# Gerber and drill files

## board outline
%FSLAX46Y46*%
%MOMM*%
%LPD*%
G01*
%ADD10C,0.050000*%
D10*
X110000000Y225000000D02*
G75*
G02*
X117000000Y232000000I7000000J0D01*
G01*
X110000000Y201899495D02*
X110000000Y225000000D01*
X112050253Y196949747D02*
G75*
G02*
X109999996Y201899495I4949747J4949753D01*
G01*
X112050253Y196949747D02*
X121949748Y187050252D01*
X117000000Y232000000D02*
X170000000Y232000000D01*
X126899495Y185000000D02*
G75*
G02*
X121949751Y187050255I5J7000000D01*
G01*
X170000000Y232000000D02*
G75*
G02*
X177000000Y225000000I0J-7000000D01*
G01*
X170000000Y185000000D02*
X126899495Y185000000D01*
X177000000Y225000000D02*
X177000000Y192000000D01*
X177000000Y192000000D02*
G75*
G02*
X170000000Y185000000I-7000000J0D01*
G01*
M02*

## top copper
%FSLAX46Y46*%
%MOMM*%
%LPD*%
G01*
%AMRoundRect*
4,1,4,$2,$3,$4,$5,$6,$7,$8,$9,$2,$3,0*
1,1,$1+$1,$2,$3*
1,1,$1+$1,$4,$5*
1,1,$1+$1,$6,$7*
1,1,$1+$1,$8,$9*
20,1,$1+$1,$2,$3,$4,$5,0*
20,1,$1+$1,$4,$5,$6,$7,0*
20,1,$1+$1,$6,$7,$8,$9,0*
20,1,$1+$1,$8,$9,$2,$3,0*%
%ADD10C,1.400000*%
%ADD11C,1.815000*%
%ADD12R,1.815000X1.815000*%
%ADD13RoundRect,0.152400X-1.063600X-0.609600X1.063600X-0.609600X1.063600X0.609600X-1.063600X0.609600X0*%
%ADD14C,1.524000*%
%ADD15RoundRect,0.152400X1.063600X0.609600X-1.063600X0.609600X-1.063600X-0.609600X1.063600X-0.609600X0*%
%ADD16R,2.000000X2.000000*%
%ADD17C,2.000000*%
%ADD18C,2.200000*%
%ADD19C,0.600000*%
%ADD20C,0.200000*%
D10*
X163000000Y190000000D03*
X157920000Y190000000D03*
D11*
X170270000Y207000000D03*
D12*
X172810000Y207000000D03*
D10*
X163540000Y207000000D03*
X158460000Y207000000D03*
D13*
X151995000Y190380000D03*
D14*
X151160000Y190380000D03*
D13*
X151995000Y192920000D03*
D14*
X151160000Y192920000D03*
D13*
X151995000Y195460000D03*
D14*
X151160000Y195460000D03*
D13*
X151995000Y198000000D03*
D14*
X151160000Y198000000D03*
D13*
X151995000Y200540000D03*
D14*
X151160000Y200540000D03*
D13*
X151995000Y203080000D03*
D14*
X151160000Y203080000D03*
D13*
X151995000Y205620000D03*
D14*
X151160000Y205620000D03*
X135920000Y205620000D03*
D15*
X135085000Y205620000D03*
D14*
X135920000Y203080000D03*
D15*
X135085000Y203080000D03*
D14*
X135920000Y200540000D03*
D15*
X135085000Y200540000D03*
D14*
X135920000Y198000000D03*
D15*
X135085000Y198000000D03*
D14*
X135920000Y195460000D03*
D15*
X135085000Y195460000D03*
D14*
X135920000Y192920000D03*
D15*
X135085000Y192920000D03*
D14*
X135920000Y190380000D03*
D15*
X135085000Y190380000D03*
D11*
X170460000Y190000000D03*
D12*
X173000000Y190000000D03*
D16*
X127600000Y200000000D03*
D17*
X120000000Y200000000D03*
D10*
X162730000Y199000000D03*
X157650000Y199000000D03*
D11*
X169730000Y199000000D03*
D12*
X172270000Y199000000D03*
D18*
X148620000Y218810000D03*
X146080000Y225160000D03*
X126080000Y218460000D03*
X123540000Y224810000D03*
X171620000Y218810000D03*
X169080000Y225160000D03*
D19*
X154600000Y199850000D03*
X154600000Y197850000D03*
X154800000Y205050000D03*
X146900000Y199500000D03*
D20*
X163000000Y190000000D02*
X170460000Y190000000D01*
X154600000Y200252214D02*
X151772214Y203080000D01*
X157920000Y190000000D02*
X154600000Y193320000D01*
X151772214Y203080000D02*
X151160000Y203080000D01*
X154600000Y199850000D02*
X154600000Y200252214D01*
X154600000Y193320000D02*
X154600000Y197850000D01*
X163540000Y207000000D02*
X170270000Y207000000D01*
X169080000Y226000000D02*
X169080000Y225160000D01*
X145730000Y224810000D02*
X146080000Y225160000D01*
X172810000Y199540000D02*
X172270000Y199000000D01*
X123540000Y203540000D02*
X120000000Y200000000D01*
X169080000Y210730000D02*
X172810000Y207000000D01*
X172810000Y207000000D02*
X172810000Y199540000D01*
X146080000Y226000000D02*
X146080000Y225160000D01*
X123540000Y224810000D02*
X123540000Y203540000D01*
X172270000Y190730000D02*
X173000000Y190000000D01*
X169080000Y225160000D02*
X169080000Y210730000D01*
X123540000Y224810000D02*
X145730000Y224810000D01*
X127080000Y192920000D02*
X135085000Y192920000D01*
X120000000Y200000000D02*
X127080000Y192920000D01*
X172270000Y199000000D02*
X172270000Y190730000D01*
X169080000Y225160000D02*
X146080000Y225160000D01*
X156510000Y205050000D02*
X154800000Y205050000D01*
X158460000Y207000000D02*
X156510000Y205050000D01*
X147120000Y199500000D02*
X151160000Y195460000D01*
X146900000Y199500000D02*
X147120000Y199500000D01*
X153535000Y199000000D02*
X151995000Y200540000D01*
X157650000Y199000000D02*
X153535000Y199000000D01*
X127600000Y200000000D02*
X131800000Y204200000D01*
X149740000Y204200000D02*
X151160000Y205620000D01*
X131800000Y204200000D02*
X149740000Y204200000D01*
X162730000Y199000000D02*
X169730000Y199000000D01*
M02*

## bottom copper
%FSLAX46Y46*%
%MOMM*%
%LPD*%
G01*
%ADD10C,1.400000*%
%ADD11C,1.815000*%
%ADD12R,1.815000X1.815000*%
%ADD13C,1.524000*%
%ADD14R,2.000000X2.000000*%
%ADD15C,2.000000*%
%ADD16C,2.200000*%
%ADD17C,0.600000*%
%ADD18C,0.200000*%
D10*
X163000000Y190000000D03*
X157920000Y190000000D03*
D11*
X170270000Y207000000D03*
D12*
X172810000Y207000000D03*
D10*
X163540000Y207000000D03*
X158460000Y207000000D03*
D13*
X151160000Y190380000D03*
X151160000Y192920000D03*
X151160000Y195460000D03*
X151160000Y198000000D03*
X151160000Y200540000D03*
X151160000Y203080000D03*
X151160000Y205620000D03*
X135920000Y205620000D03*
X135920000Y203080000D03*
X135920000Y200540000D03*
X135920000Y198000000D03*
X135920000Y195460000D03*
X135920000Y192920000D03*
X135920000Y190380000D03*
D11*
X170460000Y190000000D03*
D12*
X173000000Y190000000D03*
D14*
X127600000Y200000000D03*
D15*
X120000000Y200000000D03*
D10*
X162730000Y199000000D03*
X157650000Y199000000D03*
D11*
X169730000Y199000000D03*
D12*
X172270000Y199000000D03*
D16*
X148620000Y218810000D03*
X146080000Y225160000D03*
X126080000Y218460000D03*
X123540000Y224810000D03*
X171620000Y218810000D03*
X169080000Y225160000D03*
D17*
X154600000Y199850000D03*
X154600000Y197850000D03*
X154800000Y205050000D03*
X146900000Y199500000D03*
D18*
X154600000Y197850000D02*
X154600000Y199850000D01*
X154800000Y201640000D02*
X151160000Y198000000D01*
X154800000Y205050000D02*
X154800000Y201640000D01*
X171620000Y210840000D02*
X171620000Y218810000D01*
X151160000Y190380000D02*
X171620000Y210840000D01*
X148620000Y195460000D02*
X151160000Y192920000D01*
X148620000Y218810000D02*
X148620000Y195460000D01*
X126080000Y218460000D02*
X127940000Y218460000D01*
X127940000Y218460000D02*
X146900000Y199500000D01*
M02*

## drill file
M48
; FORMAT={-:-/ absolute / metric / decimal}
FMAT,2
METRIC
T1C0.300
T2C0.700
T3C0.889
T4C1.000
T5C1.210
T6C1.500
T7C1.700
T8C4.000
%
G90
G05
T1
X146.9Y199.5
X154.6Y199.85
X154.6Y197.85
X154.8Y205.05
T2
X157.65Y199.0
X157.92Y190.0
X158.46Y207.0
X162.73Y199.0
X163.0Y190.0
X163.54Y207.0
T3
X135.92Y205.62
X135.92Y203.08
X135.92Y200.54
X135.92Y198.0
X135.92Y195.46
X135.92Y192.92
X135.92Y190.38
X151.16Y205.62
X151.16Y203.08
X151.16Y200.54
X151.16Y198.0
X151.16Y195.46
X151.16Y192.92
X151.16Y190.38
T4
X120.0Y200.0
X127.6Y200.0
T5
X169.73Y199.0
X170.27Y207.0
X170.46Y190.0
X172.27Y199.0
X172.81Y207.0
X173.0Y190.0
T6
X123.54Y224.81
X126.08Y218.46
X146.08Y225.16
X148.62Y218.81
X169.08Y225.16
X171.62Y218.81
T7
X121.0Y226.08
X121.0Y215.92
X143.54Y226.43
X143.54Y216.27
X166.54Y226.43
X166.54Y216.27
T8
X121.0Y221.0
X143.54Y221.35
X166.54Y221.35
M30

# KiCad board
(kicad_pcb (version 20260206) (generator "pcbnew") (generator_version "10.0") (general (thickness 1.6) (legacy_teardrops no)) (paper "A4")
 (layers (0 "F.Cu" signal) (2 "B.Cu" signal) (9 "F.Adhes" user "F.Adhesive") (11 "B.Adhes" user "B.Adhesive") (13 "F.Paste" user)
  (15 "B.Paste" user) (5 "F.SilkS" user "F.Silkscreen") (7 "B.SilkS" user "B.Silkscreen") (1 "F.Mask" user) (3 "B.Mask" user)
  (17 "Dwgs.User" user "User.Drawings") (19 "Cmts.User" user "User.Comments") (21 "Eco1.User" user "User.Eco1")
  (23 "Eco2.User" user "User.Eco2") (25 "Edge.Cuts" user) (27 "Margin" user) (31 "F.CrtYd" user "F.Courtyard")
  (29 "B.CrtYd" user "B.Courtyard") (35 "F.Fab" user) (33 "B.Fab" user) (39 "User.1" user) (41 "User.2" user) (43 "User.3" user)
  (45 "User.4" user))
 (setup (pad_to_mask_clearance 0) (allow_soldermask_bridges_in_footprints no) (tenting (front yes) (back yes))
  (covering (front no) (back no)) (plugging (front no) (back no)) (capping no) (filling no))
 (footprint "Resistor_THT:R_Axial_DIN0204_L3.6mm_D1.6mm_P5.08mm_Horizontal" (layer "F.Cu") (at 163 -190 180)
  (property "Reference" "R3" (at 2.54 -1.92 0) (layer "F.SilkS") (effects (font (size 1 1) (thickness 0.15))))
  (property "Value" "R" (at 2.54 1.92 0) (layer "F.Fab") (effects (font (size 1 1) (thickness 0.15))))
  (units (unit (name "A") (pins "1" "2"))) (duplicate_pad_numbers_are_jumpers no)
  (pad "1" thru_hole circle (at 0 0 180) (size 1.4 1.4) (drill 0.7) (layers "*.Cu" "*.Mask") (remove_unused_layers no) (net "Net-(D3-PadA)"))
  (pad "2" thru_hole circle (at 5.08 0 180) (size 1.4 1.4) (drill 0.7) (layers "*.Cu" "*.Mask") (remove_unused_layers no) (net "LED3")))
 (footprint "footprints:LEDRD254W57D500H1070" (layer "F.Cu") (at 171.54 -207 180)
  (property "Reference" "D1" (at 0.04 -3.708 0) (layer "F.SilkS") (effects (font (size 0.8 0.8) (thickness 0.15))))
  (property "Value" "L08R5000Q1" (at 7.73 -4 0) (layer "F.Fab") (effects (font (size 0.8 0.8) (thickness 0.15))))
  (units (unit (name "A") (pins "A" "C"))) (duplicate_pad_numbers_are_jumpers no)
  (pad "A" thru_hole circle (at 1.27 0 180) (size 1.815 1.815) (drill 1.21) (layers "*.Cu" "*.Mask") (remove_unused_layers no)
   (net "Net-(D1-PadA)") (solder_mask_margin 0.102))
  (pad "C" thru_hole rect (at -1.27 0 180) (size 1.815 1.815) (drill 1.21) (layers "*.Cu" "*.Mask") (remove_unused_layers no) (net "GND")
   (solder_mask_margin 0.102)))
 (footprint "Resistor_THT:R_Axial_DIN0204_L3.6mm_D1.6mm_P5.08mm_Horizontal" (layer "F.Cu") (at 163.54 -207 180)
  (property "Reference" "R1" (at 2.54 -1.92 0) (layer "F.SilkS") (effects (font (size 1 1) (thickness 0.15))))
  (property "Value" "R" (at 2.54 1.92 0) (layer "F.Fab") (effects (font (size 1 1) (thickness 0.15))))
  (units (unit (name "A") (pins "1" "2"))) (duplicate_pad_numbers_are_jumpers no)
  (pad "1" thru_hole circle (at 0 0 180) (size 1.4 1.4) (drill 0.7) (layers "*.Cu" "*.Mask") (remove_unused_layers no) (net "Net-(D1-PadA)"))
  (pad "2" thru_hole circle (at 5.08 0 180) (size 1.4 1.4) (drill 0.7) (layers "*.Cu" "*.Mask") (remove_unused_layers no) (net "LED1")))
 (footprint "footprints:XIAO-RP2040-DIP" (layer "F.Cu") (at 143.54 -198 -90)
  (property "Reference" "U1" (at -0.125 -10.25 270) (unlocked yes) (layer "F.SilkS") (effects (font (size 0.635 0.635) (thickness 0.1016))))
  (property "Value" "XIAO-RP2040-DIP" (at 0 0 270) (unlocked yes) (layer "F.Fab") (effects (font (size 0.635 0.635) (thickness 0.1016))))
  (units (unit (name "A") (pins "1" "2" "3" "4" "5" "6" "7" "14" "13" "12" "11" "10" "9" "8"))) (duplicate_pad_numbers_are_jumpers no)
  (pad "1" smd roundrect (at 7.62 -8.455) (size 2.432 1.524) (layers "F.Cu" "F.Mask") (roundrect_rratio 0.1) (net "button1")
   (thermal_bridge_angle 45))
  (pad "1" thru_hole circle (at 7.62 -7.62) (size 1.524 1.524) (drill 0.889) (layers "*.Cu" "*.Mask") (remove_unused_layers no)
   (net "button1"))
  (pad "2" smd roundrect (at 5.08 -8.455) (size 2.432 1.524) (layers "F.Cu" "F.Mask") (roundrect_rratio 0.1) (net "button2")
   (thermal_bridge_angle 45))
  (pad "2" thru_hole circle (at 5.08 -7.62) (size 1.524 1.524) (drill 0.889) (layers "*.Cu" "*.Mask") (remove_unused_layers no)
   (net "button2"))
  (pad "3" smd roundrect (at 2.54 -8.455) (size 2.432 1.524) (layers "F.Cu" "F.Mask") (roundrect_rratio 0.1) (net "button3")
   (thermal_bridge_angle 45))
  (pad "3" thru_hole circle (at 2.54 -7.62) (size 1.524 1.524) (drill 0.889) (layers "*.Cu" "*.Mask") (remove_unused_layers no)
   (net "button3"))
  (pad "4" smd roundrect (at 0 -8.455) (size 2.432 1.524) (layers "F.Cu" "F.Mask") (roundrect_rratio 0.1) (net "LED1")
   (thermal_bridge_angle 45))
  (pad "4" thru_hole circle (at 0 -7.62) (size 1.524 1.524) (drill 0.889) (layers "*.Cu" "*.Mask") (remove_unused_layers no) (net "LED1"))
  (pad "5" smd roundrect (at -2.54 -8.455) (size 2.432 1.524) (layers "F.Cu" "F.Mask") (roundrect_rratio 0.1) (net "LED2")
   (thermal_bridge_angle 45))
  (pad "5" thru_hole circle (at -2.54 -7.62) (size 1.524 1.524) (drill 0.889) (layers "*.Cu" "*.Mask") (remove_unused_layers no)
   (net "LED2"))
  (pad "6" smd roundrect (at -5.08 -8.455) (size 2.432 1.524) (layers "F.Cu" "F.Mask") (roundrect_rratio 0.1) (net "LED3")
   (thermal_bridge_angle 45))
  (pad "6" thru_hole circle (at -5.08 -7.62) (size 1.524 1.524) (drill 0.889) (layers "*.Cu" "*.Mask") (remove_unused_layers no)
   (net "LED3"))
  (pad "7" smd roundrect (at -7.62 -8.455) (size 2.432 1.524) (layers "F.Cu" "F.Mask") (roundrect_rratio 0.1) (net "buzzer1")
   (thermal_bridge_angle 45))
  (pad "7" thru_hole circle (at -7.62 -7.62) (size 1.524 1.524) (drill 0.889) (layers "*.Cu" "*.Mask") (remove_unused_layers no)
   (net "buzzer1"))
  (pad "8" thru_hole circle (at -7.62 7.62 180) (size 1.524 1.524) (drill 0.889) (layers "*.Cu" "*.Mask") (remove_unused_layers no)
   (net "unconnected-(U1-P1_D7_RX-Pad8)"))
  (pad "8" smd roundrect (at -7.62 8.455 180) (size 2.432 1.524) (layers "F.Cu" "F.Mask") (roundrect_rratio 0.1)
   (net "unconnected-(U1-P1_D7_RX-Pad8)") (thermal_bridge_angle 45))
  (pad "9" thru_hole circle (at -5.08 7.62 180) (size 1.524 1.524) (drill 0.889) (layers "*.Cu" "*.Mask") (remove_unused_layers no)
   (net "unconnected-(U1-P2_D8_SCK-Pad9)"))
  (pad "9" smd roundrect (at -5.08 8.455 180) (size 2.432 1.524) (layers "F.Cu" "F.Mask") (roundrect_rratio 0.1)
   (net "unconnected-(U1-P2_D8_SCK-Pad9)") (thermal_bridge_angle 45))
  (pad "10" thru_hole circle (at -2.54 7.62 180) (size 1.524 1.524) (drill 0.889) (layers "*.Cu" "*.Mask") (remove_unused_layers no)
   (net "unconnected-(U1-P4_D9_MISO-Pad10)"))
  (pad "10" smd roundrect (at -2.54 8.455 180) (size 2.432 1.524) (layers "F.Cu" "F.Mask") (roundrect_rratio 0.1)
   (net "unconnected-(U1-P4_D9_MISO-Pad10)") (thermal_bridge_angle 45))
  (pad "11" thru_hole circle (at 0 7.62 180) (size 1.524 1.524) (drill 0.889) (layers "*.Cu" "*.Mask") (remove_unused_layers no)
   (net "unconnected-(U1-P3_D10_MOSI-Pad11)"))
  (pad "11" smd roundrect (at 0 8.455 180) (size 2.432 1.524) (layers "F.Cu" "F.Mask") (roundrect_rratio 0.1)
   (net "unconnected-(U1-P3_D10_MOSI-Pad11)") (thermal_bridge_angle 45))
  (pad "12" thru_hole circle (at 2.54 7.62 180) (size 1.524 1.524) (drill 0.889) (layers "*.Cu" "*.Mask") (remove_unused_layers no)
   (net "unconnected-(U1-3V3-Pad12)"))
  (pad "12" smd roundrect (at 2.54 8.455 180) (size 2.432 1.524) (layers "F.Cu" "F.Mask") (roundrect_rratio 0.1)
   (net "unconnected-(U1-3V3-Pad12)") (thermal_bridge_angle 45))
  (pad "13" thru_hole circle (at 5.08 7.62 180) (size 1.524 1.524) (drill 0.889) (layers "*.Cu" "*.Mask") (remove_unused_layers no)
   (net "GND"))
  (pad "13" smd roundrect (at 5.08 8.455 180) (size 2.432 1.524) (layers "F.Cu" "F.Mask") (roundrect_rratio 0.1) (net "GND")
   (thermal_bridge_angle 45))
  (pad "14" thru_hole circle (at 7.62 7.62 180) (size 1.524 1.524) (drill 0.889) (layers "*.Cu" "*.Mask") (remove_unused_layers no)
   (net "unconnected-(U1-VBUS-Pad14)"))
  (pad "14" smd roundrect (at 7.62 8.455 180) (size 2.432 1.524) (layers "F.Cu" "F.Mask") (roundrect_rratio 0.1)
   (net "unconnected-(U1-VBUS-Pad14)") (thermal_bridge_angle 45)))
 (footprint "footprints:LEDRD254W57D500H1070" (layer "F.Cu") (at 171.73 -190 180)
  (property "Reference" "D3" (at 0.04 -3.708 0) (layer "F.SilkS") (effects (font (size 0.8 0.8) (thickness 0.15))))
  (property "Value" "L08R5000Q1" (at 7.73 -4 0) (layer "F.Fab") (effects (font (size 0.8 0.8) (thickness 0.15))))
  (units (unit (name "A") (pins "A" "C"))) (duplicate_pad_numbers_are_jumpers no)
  (pad "A" thru_hole circle (at 1.27 0 180) (size 1.815 1.815) (drill 1.21) (layers "*.Cu" "*.Mask") (remove_unused_layers no)
   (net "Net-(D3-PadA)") (solder_mask_margin 0.102))
  (pad "C" thru_hole rect (at -1.27 0 180) (size 1.815 1.815) (drill 1.21) (layers "*.Cu" "*.Mask") (remove_unused_layers no) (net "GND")
   (solder_mask_margin 0.102)))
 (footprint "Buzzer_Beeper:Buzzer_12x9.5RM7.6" (layer "F.Cu") (at 127.6 -200 180)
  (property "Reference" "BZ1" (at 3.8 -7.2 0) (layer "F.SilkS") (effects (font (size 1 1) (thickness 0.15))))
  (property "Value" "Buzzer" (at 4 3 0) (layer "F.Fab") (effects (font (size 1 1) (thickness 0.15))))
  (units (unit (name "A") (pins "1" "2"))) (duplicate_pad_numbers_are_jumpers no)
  (pad "1" thru_hole rect (at 0 0 180) (size 2 2) (drill 1) (layers "*.Cu" "*.Mask") (remove_unused_layers no) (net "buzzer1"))
  (pad "2" thru_hole circle (at 7.6 0 180) (size 2 2) (drill 1) (layers "*.Cu" "*.Mask") (remove_unused_layers no) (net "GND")))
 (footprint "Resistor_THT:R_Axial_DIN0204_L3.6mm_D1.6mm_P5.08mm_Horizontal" (layer "F.Cu") (at 162.73 -199 180)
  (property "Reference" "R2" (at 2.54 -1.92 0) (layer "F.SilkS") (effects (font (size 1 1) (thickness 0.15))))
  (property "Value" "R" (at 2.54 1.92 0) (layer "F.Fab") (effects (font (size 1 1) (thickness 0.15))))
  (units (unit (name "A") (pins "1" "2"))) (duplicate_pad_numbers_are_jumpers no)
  (pad "1" thru_hole circle (at 0 0 180) (size 1.4 1.4) (drill 0.7) (layers "*.Cu" "*.Mask") (remove_unused_layers no) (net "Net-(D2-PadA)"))
  (pad "2" thru_hole circle (at 5.08 0 180) (size 1.4 1.4) (drill 0.7) (layers "*.Cu" "*.Mask") (remove_unused_layers no) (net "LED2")))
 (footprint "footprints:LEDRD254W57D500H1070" (layer "F.Cu") (at 171 -199 180)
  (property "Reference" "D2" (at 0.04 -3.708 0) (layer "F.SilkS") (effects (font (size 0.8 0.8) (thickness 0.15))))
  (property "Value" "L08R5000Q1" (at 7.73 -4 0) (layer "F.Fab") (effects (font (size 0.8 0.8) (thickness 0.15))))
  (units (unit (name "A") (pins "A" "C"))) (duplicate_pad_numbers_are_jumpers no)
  (pad "A" thru_hole circle (at 1.27 0 180) (size 1.815 1.815) (drill 1.21) (layers "*.Cu" "*.Mask") (remove_unused_layers no)
   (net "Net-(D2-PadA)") (solder_mask_margin 0.102))
  (pad "C" thru_hole rect (at -1.27 0 180) (size 1.815 1.815) (drill 1.21) (layers "*.Cu" "*.Mask") (remove_unused_layers no) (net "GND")
   (solder_mask_margin 0.102)))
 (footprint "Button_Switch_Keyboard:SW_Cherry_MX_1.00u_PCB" (layer "F.Cu") (at 148.62 -218.81 -90)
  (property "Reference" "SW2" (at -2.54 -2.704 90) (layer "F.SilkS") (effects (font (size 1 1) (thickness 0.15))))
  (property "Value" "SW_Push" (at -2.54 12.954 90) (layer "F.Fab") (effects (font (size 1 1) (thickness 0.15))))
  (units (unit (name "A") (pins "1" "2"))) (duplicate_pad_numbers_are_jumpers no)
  (pad "" np_thru_hole circle (at -7.62 5.08 270) (size 1.7 1.7) (drill 1.7) (layers "*.Cu" "*.Mask"))
  (pad "" np_thru_hole circle (at -2.54 5.08 270) (size 4 4) (drill 4) (layers "*.Cu" "*.Mask"))
  (pad "" np_thru_hole circle (at 2.54 5.08 270) (size 1.7 1.7) (drill 1.7) (layers "*.Cu" "*.Mask"))
  (pad "1" thru_hole circle (at 0 0 270) (size 2.2 2.2) (drill 1.5) (layers "*.Cu" "*.Mask") (remove_unused_layers no) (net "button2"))
  (pad "2" thru_hole circle (at -6.35 2.54 270) (size 2.2 2.2) (drill 1.5) (layers "*.Cu" "*.Mask") (remove_unused_layers no) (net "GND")))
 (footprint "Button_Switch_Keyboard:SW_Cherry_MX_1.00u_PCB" (layer "F.Cu") (at 126.08 -218.46 -90)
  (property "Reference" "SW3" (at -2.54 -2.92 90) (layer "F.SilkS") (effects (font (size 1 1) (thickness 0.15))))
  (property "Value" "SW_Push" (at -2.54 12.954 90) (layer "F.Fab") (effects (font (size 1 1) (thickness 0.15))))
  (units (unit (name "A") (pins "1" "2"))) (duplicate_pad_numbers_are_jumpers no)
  (pad "" np_thru_hole circle (at -7.62 5.08 270) (size 1.7 1.7) (drill 1.7) (layers "*.Cu" "*.Mask"))
  (pad "" np_thru_hole circle (at -2.54 5.08 270) (size 4 4) (drill 4) (layers "*.Cu" "*.Mask"))
  (pad "" np_thru_hole circle (at 2.54 5.08 270) (size 1.7 1.7) (drill 1.7) (layers "*.Cu" "*.Mask"))
  (pad "1" thru_hole circle (at 0 0 270) (size 2.2 2.2) (drill 1.5) (layers "*.Cu" "*.Mask") (remove_unused_layers no) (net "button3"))
  (pad "2" thru_hole circle (at -6.35 2.54 270) (size 2.2 2.2) (drill 1.5) (layers "*.Cu" "*.Mask") (remove_unused_layers no) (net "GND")))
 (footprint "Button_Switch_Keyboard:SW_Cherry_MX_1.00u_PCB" (layer "F.Cu") (at 171.62 -218.81 -90)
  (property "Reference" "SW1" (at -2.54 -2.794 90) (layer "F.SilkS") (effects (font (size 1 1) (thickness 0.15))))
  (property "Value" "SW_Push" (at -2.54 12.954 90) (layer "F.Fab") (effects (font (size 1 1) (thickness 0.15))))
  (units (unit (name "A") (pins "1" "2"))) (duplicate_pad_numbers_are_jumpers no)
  (pad "" np_thru_hole circle (at -7.62 5.08 270) (size 1.7 1.7) (drill 1.7) (layers "*.Cu" "*.Mask"))
  (pad "" np_thru_hole circle (at -2.54 5.08 270) (size 4 4) (drill 4) (layers "*.Cu" "*.Mask"))
  (pad "" np_thru_hole circle (at 2.54 5.08 270) (size 1.7 1.7) (drill 1.7) (layers "*.Cu" "*.Mask"))
  (pad "1" thru_hole circle (at 0 0 270) (size 2.2 2.2) (drill 1.5) (layers "*.Cu" "*.Mask") (remove_unused_layers no) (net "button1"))
  (pad "2" thru_hole circle (at -6.35 2.54 270) (size 2.2 2.2) (drill 1.5) (layers "*.Cu" "*.Mask") (remove_unused_layers no) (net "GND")))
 (gr_arc (start 110 -225) (mid 112.050253 -229.949747) (end 117 -232) (stroke (width 0.05) (type default)) (layer "Edge.Cuts"))
 (gr_line (start 110 -201.899495) (end 110 -225) (stroke (width 0.05) (type default)) (layer "Edge.Cuts"))
 (gr_arc (start 112.050253 -196.949747) (mid 110.532842 -199.22071) (end 110 -201.899495) (stroke (width 0.05) (type default))
  (layer "Edge.Cuts"))
 (gr_line (start 112.050253 -196.949747) (end 121.949748 -187.050252) (stroke (width 0.05) (type default)) (layer "Edge.Cuts"))
 (gr_line (start 117 -232) (end 170 -232) (stroke (width 0.05) (type default)) (layer "Edge.Cuts"))
 (gr_arc (start 126.899495 -185) (mid 124.220711 -185.532843) (end 121.949748 -187.050252) (stroke (width 0.05) (type default))
  (layer "Edge.Cuts"))
 (gr_arc (start 170 -232) (mid 174.949747 -229.949747) (end 177 -225) (stroke (width 0.05) (type default)) (layer "Edge.Cuts"))
 (gr_line (start 170 -185) (end 126.899495 -185) (stroke (width 0.05) (type default)) (layer "Edge.Cuts"))
 (gr_line (start 177 -225) (end 177 -192) (stroke (width 0.05) (type default)) (layer "Edge.Cuts"))
 (gr_arc (start 177 -192) (mid 174.949747 -187.050253) (end 170 -185) (stroke (width 0.05) (type default)) (layer "Edge.Cuts"))
 (segment (start 163 -190) (end 170.46 -190) (width 0.2) (layer "F.Cu") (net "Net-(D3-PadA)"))
 (segment (start 154.6 -200.252214) (end 151.772214 -203.08) (width 0.2) (layer "F.Cu") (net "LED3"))
 (segment (start 157.92 -190) (end 154.6 -193.32) (width 0.2) (layer "F.Cu") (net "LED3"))
 (segment (start 151.772214 -203.08) (end 151.16 -203.08) (width 0.2) (layer "F.Cu") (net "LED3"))
 (segment (start 154.6 -199.85) (end 154.6 -200.252214) (width 0.2) (layer "F.Cu") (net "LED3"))
 (segment (start 154.6 -193.32) (end 154.6 -197.85) (width 0.2) (layer "F.Cu") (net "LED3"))
 (via (at 154.6 -199.85) (size 0.6) (drill 0.3) (layers "F.Cu" "B.Cu") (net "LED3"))
 (via (at 154.6 -197.85) (size 0.6) (drill 0.3) (layers "F.Cu" "B.Cu") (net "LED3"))
 (segment (start 154.6 -197.85) (end 154.6 -199.85) (width 0.2) (layer "B.Cu") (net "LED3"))
 (segment (start 163.54 -207) (end 170.27 -207) (width 0.2) (layer "F.Cu") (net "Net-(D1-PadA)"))
 (segment (start 169.08 -226) (end 169.08 -225.16) (width 0.2) (layer "F.Cu") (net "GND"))
 (segment (start 145.73 -224.81) (end 146.08 -225.16) (width 0.2) (layer "F.Cu") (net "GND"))
 (segment (start 172.81 -199.54) (end 172.27 -199) (width 0.2) (layer "F.Cu") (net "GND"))
 (segment (start 123.54 -203.54) (end 120 -200) (width 0.2) (layer "F.Cu") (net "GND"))
 (segment (start 169.08 -210.73) (end 172.81 -207) (width 0.2) (layer "F.Cu") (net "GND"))
 (segment (start 172.81 -207) (end 172.81 -199.54) (width 0.2) (layer "F.Cu") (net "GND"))
 (segment (start 146.08 -226) (end 146.08 -225.16) (width 0.2) (layer "F.Cu") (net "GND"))
 (segment (start 123.54 -224.81) (end 123.54 -203.54) (width 0.2) (layer "F.Cu") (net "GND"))
 (segment (start 172.27 -190.73) (end 173 -190) (width 0.2) (layer "F.Cu") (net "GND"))
 (segment (start 169.08 -225.16) (end 169.08 -210.73) (width 0.2) (layer "F.Cu") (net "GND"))
 (segment (start 123.54 -224.81) (end 145.73 -224.81) (width 0.2) (layer "F.Cu") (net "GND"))
 (segment (start 127.08 -192.92) (end 135.085 -192.92) (width 0.2) (layer "F.Cu") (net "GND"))
 (segment (start 120 -200) (end 127.08 -192.92) (width 0.2) (layer "F.Cu") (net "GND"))
 (segment (start 172.27 -199) (end 172.27 -190.73) (width 0.2) (layer "F.Cu") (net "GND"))
 (segment (start 169.08 -225.16) (end 146.08 -225.16) (width 0.2) (layer "F.Cu") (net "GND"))
 (segment (start 156.51 -205.05) (end 154.8 -205.05) (width 0.2) (layer "F.Cu") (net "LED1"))
 (segment (start 158.46 -207) (end 156.51 -205.05) (width 0.2) (layer "F.Cu") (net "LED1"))
 (via (at 154.8 -205.05) (size 0.6) (drill 0.3) (layers "F.Cu" "B.Cu") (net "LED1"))
 (segment (start 154.8 -201.64) (end 151.16 -198) (width 0.2) (layer "B.Cu") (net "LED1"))
 (segment (start 154.8 -205.05) (end 154.8 -201.64) (width 0.2) (layer "B.Cu") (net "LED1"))
 (segment (start 171.62 -210.84) (end 171.62 -218.81) (width 0.2) (layer "B.Cu") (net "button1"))
 (segment (start 151.16 -190.38) (end 171.62 -210.84) (width 0.2) (layer "B.Cu") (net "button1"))
 (segment (start 148.62 -195.46) (end 151.16 -192.92) (width 0.2) (layer "B.Cu") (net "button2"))
 (segment (start 148.62 -218.81) (end 148.62 -195.46) (width 0.2) (layer "B.Cu") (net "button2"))
 (segment (start 147.12 -199.5) (end 151.16 -195.46) (width 0.2) (layer "F.Cu") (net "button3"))
 (segment (start 146.9 -199.5) (end 147.12 -199.5) (width 0.2) (layer "F.Cu") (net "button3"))
 (via (at 146.9 -199.5) (size 0.6) (drill 0.3) (layers "F.Cu" "B.Cu") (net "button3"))
 (segment (start 126.08 -218.46) (end 127.94 -218.46) (width 0.2) (layer "B.Cu") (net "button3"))
 (segment (start 127.94 -218.46) (end 146.9 -199.5) (width 0.2) (layer "B.Cu") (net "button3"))
 (segment (start 153.535 -199) (end 151.995 -200.54) (width 0.2) (layer "F.Cu") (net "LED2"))
 (segment (start 157.65 -199) (end 153.535 -199) (width 0.2) (layer "F.Cu") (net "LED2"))
 (segment (start 127.6 -200) (end 131.8 -204.2) (width 0.2) (layer "F.Cu") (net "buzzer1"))
 (segment (start 149.74 -204.2) (end 151.16 -205.62) (width 0.2) (layer "F.Cu") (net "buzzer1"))
 (segment (start 131.8 -204.2) (end 149.74 -204.2) (width 0.2) (layer "F.Cu") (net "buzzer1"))
 (segment (start 162.73 -199) (end 169.73 -199) (width 0.2) (layer "F.Cu") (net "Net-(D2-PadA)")))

